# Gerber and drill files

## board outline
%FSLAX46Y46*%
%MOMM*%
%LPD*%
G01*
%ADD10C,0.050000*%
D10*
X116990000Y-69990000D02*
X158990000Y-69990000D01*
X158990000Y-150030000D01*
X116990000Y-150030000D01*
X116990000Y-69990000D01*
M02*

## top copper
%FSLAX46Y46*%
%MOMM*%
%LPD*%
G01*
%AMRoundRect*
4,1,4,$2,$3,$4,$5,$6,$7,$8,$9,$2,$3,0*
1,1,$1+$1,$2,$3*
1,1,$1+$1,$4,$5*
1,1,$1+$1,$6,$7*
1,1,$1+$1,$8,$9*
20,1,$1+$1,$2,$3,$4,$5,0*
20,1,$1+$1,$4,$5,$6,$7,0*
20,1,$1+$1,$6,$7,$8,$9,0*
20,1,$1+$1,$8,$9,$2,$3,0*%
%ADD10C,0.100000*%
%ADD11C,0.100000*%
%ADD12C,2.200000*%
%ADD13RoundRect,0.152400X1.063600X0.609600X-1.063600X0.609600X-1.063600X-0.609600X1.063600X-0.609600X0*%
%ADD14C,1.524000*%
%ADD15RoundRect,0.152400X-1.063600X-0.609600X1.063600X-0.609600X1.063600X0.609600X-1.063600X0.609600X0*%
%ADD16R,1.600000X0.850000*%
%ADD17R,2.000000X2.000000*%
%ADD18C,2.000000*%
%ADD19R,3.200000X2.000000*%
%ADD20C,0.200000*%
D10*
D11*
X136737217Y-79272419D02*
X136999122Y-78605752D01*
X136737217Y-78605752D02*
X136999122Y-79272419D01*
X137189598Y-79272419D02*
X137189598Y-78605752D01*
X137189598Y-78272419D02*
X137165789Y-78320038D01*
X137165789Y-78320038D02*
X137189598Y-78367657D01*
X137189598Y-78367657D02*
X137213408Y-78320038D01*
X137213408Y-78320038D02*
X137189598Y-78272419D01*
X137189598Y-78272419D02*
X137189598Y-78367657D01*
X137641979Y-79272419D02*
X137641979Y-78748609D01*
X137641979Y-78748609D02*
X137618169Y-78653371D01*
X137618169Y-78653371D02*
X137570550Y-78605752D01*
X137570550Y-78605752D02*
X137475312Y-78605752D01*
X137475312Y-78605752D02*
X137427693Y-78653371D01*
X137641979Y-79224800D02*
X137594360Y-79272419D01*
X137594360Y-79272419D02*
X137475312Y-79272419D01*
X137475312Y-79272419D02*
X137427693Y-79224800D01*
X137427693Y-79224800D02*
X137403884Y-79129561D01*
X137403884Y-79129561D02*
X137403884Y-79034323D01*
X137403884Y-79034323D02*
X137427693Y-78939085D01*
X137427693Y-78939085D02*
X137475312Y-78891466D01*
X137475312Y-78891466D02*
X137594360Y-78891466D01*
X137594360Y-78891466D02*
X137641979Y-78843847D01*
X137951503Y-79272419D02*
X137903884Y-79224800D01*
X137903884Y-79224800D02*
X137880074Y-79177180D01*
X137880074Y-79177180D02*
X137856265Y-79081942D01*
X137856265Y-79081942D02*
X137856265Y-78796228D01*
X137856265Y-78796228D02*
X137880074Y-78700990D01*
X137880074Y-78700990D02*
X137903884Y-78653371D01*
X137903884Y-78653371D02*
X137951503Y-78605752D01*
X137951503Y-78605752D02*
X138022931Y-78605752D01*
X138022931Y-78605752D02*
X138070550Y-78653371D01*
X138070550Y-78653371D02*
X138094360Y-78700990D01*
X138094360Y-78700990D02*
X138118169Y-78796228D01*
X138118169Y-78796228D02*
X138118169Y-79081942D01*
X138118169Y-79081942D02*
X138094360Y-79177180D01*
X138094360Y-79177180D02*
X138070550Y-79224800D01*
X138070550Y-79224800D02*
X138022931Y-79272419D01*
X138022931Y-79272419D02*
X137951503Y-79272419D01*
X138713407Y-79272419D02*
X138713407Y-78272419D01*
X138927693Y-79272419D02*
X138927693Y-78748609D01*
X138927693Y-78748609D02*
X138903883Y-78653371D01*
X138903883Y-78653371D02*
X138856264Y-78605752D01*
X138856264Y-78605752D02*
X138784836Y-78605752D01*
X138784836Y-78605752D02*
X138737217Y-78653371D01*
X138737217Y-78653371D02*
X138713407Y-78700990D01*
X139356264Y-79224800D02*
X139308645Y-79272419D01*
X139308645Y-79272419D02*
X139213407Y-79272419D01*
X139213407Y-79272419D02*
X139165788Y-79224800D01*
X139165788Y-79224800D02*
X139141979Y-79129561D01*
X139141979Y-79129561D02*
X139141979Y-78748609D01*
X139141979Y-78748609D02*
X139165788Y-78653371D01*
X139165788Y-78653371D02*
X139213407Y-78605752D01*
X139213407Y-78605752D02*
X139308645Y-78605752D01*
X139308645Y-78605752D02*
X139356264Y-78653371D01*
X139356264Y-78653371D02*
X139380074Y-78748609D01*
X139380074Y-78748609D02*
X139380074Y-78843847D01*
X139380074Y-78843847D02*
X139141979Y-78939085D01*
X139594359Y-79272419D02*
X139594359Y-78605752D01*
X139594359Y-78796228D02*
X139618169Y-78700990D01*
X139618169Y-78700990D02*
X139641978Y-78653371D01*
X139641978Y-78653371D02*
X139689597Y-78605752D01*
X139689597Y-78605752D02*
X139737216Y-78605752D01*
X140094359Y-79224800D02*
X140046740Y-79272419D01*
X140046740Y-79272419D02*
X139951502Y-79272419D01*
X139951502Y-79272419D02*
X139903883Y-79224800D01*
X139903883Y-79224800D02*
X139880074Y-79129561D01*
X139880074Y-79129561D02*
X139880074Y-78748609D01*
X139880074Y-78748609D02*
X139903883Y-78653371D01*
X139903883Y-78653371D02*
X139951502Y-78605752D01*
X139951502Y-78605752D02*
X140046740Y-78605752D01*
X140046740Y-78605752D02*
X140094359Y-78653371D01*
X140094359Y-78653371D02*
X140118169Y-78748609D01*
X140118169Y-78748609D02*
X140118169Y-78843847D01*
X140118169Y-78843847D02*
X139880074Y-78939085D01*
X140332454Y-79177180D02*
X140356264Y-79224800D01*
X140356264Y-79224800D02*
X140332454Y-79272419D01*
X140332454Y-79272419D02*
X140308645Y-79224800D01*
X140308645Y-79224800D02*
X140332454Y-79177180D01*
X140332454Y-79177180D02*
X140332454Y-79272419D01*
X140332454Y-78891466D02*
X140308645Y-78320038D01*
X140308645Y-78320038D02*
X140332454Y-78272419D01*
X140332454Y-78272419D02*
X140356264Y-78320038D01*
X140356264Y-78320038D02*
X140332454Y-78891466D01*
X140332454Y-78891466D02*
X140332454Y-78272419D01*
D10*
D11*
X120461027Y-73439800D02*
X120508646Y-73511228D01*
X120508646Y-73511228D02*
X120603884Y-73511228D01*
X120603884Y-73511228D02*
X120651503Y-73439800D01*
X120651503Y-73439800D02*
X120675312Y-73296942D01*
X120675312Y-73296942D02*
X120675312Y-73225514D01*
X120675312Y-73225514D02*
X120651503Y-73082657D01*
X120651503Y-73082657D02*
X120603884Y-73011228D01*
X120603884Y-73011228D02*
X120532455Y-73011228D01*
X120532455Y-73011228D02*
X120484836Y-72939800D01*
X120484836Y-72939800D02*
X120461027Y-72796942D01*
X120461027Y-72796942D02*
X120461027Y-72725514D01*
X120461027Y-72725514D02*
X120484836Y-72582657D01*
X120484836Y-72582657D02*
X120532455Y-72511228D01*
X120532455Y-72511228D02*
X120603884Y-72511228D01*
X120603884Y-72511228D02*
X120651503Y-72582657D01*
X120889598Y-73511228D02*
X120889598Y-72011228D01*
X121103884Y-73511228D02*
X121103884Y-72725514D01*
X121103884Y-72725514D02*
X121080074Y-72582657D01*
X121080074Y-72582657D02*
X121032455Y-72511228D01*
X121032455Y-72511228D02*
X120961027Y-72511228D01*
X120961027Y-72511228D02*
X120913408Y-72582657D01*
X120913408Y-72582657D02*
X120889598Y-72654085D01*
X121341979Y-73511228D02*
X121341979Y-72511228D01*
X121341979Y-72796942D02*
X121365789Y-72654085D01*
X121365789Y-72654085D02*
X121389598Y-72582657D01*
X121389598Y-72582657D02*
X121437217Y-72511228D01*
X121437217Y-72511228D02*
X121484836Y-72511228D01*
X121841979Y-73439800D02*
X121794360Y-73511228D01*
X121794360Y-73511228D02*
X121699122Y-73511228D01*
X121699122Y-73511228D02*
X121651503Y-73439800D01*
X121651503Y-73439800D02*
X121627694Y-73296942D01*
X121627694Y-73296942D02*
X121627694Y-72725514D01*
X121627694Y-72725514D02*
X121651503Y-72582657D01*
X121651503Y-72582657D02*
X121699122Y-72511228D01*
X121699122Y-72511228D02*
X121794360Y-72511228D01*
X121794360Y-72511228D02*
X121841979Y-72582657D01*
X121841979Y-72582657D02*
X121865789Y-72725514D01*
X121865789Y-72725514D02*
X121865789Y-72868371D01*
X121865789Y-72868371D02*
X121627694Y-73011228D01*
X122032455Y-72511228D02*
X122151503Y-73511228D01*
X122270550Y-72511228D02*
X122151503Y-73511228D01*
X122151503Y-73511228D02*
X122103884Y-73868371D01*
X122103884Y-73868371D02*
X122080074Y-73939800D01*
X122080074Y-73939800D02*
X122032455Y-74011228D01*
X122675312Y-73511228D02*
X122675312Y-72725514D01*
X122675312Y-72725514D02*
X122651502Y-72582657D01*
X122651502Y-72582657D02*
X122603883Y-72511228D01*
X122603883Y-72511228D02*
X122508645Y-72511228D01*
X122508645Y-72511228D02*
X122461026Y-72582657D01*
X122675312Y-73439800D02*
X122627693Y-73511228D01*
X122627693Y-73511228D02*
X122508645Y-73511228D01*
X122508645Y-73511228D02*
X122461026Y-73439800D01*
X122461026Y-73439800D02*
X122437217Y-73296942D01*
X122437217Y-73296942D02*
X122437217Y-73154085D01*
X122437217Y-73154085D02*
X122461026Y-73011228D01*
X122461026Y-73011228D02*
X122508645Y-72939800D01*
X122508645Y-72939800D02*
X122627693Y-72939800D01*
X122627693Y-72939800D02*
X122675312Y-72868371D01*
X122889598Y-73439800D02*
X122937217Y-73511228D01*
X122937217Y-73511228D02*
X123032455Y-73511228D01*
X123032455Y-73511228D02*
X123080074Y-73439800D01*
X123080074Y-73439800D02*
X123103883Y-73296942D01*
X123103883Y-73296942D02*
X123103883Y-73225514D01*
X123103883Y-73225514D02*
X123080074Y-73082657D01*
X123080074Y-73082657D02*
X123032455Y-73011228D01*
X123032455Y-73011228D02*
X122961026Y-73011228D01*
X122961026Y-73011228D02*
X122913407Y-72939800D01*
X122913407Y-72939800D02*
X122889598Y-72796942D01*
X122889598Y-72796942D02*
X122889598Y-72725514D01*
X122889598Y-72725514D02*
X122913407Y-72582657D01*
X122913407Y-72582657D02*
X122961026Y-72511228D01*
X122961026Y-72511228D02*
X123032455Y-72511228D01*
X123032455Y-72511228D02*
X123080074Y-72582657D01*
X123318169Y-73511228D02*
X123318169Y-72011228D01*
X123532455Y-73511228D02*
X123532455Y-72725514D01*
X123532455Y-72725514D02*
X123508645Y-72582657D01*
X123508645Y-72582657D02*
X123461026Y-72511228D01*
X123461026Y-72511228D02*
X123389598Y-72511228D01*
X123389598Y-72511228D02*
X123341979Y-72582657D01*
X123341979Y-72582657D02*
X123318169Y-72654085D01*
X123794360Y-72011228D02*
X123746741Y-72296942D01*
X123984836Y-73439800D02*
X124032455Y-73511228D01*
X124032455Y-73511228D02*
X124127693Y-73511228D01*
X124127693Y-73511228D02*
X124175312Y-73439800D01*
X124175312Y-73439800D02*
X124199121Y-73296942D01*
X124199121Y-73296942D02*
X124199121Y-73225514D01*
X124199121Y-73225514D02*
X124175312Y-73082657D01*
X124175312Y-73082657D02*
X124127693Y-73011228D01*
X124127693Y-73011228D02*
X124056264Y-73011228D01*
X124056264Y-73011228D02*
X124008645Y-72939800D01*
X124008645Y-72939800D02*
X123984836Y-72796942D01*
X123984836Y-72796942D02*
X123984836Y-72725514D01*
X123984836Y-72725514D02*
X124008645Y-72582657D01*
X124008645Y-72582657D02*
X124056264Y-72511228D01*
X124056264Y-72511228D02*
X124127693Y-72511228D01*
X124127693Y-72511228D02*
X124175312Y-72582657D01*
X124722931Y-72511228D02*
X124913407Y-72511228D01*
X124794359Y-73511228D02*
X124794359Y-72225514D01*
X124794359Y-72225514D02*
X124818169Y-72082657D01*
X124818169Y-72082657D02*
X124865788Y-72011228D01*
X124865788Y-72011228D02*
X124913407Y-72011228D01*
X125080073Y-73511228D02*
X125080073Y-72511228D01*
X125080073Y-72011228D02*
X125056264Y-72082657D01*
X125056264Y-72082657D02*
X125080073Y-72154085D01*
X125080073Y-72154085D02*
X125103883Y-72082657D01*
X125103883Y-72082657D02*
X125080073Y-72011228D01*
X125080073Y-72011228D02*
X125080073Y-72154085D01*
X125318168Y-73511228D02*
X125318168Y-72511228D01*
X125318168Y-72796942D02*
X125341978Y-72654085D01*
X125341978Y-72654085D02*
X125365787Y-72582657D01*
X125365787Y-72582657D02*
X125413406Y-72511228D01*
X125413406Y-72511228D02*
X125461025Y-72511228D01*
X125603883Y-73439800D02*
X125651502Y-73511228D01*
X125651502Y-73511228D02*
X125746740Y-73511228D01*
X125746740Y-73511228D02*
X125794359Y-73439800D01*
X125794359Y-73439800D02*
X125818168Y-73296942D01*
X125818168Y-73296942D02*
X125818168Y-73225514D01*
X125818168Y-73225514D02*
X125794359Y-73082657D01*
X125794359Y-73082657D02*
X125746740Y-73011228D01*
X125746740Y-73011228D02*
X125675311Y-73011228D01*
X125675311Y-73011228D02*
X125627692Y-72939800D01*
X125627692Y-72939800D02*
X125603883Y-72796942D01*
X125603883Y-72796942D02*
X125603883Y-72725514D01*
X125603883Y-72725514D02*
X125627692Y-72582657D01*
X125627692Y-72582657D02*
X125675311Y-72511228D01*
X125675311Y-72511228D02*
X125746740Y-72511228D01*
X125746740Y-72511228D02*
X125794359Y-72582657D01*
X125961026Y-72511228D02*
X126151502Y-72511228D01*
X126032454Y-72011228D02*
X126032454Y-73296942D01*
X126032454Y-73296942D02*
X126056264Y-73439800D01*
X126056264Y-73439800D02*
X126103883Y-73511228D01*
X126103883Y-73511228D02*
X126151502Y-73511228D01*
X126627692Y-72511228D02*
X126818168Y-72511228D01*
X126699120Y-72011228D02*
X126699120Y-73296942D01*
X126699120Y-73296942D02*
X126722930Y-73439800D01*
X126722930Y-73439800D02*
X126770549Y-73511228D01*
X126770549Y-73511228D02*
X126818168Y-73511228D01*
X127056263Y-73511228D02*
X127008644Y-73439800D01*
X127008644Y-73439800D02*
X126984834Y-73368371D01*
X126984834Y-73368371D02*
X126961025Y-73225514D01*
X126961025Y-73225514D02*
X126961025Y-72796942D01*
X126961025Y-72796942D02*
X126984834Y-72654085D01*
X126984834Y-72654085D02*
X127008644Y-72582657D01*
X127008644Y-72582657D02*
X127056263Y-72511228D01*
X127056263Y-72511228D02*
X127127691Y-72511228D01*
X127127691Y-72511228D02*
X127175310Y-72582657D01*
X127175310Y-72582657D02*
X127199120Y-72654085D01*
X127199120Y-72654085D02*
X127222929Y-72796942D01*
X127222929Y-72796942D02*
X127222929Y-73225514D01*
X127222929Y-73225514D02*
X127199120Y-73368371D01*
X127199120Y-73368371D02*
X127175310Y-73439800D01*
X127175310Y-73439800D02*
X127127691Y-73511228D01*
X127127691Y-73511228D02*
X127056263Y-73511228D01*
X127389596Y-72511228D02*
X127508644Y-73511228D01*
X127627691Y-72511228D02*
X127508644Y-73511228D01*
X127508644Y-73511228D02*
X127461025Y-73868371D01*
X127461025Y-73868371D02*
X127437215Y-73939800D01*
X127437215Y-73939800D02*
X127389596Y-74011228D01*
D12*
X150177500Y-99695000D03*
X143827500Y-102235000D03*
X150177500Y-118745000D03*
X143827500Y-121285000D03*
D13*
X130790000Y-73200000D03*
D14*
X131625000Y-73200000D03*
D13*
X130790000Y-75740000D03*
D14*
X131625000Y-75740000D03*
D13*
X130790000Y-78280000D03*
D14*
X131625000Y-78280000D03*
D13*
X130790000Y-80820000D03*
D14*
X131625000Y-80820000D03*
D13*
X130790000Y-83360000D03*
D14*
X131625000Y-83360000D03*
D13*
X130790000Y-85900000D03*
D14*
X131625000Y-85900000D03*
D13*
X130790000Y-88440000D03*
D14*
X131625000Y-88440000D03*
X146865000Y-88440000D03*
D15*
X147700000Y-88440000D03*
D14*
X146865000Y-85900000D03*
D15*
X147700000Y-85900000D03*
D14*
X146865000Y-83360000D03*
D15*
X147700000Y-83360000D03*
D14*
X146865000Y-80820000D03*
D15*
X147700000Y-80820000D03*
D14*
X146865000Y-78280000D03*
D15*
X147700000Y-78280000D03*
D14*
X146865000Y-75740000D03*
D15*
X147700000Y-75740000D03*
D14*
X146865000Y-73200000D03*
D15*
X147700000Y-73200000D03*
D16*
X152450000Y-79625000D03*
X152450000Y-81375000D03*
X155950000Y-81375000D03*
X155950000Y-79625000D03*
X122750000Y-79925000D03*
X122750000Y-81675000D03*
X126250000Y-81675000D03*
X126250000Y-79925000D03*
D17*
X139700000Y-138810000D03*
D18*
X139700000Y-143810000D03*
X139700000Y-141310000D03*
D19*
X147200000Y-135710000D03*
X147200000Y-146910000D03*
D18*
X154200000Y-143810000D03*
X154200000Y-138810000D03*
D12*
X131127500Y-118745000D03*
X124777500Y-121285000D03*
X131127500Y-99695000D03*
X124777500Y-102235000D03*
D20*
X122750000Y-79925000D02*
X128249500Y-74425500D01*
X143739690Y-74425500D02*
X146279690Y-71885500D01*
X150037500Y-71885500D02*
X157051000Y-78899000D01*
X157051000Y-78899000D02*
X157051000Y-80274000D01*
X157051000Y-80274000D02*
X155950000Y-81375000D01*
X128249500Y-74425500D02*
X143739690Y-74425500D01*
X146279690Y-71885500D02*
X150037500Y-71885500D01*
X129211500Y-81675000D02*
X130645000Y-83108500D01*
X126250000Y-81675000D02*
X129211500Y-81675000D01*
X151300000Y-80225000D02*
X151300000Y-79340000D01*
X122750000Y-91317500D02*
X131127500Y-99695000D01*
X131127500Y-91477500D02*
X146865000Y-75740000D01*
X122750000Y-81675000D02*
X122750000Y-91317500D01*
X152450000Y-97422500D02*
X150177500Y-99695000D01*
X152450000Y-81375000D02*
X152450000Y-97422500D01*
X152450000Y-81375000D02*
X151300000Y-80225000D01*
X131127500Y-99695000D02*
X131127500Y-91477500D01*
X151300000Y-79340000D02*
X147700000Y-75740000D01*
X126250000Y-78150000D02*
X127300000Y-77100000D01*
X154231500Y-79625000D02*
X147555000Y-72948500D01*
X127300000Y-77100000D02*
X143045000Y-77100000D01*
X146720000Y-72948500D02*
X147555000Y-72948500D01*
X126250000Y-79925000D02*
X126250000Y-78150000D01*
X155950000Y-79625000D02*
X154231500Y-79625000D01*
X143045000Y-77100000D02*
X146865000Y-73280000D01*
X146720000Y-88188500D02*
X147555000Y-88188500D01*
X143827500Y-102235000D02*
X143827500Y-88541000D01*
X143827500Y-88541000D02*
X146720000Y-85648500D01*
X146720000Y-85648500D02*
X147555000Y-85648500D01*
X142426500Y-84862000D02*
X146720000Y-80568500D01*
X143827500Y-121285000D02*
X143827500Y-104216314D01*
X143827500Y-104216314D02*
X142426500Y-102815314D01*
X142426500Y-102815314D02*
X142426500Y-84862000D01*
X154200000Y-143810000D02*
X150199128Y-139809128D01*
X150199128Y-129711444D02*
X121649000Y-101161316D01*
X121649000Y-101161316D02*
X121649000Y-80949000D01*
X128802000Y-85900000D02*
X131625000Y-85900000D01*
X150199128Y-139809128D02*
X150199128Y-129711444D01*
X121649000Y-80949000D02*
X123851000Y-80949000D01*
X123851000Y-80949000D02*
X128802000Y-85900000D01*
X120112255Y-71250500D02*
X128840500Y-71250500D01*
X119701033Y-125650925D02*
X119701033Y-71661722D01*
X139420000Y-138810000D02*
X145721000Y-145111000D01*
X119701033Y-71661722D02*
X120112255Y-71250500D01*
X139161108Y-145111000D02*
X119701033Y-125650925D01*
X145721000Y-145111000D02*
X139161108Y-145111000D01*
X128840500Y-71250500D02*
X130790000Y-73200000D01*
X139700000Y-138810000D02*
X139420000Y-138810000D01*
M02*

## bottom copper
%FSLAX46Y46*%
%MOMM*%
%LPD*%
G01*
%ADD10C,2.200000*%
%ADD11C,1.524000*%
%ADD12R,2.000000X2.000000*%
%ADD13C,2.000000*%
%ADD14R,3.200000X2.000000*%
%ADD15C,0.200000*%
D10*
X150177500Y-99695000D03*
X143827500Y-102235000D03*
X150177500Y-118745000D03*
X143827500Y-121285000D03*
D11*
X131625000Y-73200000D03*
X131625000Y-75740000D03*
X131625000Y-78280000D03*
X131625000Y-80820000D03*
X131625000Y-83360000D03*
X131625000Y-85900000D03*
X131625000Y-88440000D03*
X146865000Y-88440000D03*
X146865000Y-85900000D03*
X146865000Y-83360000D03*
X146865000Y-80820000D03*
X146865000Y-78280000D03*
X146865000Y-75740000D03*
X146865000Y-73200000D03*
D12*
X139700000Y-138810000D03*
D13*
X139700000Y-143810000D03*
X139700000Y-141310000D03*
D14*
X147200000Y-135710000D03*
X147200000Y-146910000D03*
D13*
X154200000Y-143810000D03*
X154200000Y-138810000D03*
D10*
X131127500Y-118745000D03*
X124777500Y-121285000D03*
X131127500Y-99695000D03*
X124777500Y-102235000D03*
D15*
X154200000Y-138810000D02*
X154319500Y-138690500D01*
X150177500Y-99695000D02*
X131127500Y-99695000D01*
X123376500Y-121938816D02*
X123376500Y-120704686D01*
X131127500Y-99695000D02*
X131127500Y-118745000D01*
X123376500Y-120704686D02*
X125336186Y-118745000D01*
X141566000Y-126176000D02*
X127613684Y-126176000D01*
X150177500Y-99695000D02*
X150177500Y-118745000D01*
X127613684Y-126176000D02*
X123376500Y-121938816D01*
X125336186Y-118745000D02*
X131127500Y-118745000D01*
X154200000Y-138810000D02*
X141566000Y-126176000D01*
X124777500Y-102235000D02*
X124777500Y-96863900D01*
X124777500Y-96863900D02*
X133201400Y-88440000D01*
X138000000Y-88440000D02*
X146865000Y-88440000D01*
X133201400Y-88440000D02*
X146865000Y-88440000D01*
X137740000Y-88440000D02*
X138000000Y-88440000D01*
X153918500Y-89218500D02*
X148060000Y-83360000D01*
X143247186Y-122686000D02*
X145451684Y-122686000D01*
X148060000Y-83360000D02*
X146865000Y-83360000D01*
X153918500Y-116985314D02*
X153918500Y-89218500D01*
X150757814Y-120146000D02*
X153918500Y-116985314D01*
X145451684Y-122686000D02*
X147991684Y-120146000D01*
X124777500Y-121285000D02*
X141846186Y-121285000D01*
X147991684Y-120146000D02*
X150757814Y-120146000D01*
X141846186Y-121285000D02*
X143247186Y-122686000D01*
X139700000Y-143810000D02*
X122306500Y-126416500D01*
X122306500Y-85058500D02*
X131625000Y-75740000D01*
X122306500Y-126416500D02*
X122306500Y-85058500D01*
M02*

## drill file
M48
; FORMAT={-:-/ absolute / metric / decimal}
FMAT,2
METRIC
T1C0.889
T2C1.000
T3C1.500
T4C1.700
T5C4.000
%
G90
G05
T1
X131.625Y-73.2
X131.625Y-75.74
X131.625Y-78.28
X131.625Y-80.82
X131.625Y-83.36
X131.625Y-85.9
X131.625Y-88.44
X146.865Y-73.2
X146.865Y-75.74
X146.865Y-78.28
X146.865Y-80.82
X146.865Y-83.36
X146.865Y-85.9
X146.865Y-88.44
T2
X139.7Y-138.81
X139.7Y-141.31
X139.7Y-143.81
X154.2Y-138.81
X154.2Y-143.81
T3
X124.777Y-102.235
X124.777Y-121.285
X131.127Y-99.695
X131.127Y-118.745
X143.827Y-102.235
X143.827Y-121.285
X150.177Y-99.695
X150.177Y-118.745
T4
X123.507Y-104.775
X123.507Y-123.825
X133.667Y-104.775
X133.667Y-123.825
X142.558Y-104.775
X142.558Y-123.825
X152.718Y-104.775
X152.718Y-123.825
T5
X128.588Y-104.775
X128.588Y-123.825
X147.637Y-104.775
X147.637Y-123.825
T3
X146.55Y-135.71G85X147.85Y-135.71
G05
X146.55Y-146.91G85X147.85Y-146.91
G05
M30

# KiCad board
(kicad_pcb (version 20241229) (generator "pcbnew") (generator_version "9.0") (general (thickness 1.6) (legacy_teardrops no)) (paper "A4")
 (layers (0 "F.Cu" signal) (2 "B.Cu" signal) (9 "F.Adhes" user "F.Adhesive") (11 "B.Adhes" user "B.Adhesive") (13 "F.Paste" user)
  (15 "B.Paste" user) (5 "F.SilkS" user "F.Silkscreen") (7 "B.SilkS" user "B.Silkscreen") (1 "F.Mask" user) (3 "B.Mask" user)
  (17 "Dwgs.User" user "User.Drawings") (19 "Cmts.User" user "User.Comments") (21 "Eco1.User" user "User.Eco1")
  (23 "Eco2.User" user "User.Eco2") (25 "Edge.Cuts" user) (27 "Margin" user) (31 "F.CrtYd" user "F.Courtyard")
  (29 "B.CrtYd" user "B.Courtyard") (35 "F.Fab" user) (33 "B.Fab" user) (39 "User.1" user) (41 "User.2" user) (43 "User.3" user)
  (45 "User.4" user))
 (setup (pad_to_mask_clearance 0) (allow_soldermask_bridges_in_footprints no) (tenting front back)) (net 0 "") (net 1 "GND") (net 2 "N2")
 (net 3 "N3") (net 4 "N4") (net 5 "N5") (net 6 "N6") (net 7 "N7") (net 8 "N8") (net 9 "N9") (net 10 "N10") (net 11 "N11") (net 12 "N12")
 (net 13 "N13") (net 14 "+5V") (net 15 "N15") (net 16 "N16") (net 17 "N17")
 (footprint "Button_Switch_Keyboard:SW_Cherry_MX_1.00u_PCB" (layer "F.Cu") (at 150.1775 99.695)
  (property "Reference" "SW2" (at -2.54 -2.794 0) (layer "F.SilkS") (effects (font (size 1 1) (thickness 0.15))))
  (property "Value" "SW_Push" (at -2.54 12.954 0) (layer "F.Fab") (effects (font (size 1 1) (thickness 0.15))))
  (pad "" np_thru_hole circle (at -7.62 5.08) (size 1.7 1.7) (drill 1.7) (layers "*.Cu" "*.Mask"))
  (pad "" np_thru_hole circle (at -2.54 5.08) (size 4 4) (drill 4) (layers "*.Cu" "*.Mask"))
  (pad "" np_thru_hole circle (at 2.54 5.08) (size 1.7 1.7) (drill 1.7) (layers "*.Cu" "*.Mask"))
  (pad "1" thru_hole circle (at 0 0) (size 2.2 2.2) (drill 1.5) (layers "*.Cu" "*.Mask") (remove_unused_layers no) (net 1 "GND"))
  (pad "2" thru_hole circle (at -6.35 2.54) (size 2.2 2.2) (drill 1.5) (layers "*.Cu" "*.Mask") (remove_unused_layers no) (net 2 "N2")))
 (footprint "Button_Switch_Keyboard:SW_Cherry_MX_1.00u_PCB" (layer "F.Cu") (at 150.1775 118.745)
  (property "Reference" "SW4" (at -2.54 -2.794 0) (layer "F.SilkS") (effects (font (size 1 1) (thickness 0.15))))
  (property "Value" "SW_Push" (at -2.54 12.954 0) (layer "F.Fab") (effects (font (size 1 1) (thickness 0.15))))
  (pad "" np_thru_hole circle (at -7.62 5.08) (size 1.7 1.7) (drill 1.7) (layers "*.Cu" "*.Mask"))
  (pad "" np_thru_hole circle (at -2.54 5.08) (size 4 4) (drill 4) (layers "*.Cu" "*.Mask"))
  (pad "" np_thru_hole circle (at 2.54 5.08) (size 1.7 1.7) (drill 1.7) (layers "*.Cu" "*.Mask"))
  (pad "1" thru_hole circle (at 0 0) (size 2.2 2.2) (drill 1.5) (layers "*.Cu" "*.Mask") (remove_unused_layers no) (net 1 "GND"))
  (pad "2" thru_hole circle (at -6.35 2.54) (size 2.2 2.2) (drill 1.5) (layers "*.Cu" "*.Mask") (remove_unused_layers no) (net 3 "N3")))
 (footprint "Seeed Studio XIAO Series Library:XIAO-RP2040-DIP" (layer "F.Cu") (at 139.245 80.82)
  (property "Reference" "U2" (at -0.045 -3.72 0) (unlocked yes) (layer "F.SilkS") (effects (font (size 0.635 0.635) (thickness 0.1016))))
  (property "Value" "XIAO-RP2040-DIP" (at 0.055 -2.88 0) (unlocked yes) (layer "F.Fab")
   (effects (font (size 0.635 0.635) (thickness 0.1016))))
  (pad "1" smd roundrect (at -8.455 -7.62 180) (size 2.432 1.524) (layers "F.Cu" "F.Mask") (roundrect_rratio 0.1) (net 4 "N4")
   (thermal_bridge_angle 45))
  (pad "1" thru_hole circle (at -7.62 -7.62 180) (size 1.524 1.524) (drill 0.889) (layers "*.Cu" "*.Mask") (remove_unused_layers no)
   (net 4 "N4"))
  (pad "2" smd roundrect (at -8.455 -5.08 180) (size 2.432 1.524) (layers "F.Cu" "F.Mask") (roundrect_rratio 0.1) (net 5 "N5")
   (thermal_bridge_angle 45))
  (pad "2" thru_hole circle (at -7.62 -5.08 180) (size 1.524 1.524) (drill 0.889) (layers "*.Cu" "*.Mask") (remove_unused_layers no)
   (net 5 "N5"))
  (pad "3" smd roundrect (at -8.455 -2.54 180) (size 2.432 1.524) (layers "F.Cu" "F.Mask") (roundrect_rratio 0.1) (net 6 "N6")
   (thermal_bridge_angle 45))
  (pad "3" thru_hole circle (at -7.62 -2.54 180) (size 1.524 1.524) (drill 0.889) (layers "*.Cu" "*.Mask") (remove_unused_layers no)
   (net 6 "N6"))
  (pad "4" smd roundrect (at -8.455 0 180) (size 2.432 1.524) (layers "F.Cu" "F.Mask") (roundrect_rratio 0.1) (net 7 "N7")
   (thermal_bridge_angle 45))
  (pad "4" thru_hole circle (at -7.62 0 180) (size 1.524 1.524) (drill 0.889) (layers "*.Cu" "*.Mask") (remove_unused_layers no)
   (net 7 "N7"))
  (pad "5" smd roundrect (at -8.455 2.54 180) (size 2.432 1.524) (layers "F.Cu" "F.Mask") (roundrect_rratio 0.1) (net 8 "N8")
   (thermal_bridge_angle 45))
  (pad "5" thru_hole circle (at -7.62 2.54 180) (size 1.524 1.524) (drill 0.889) (layers "*.Cu" "*.Mask") (remove_unused_layers no)
   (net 8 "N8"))
  (pad "6" smd roundrect (at -8.455 5.08 180) (size 2.432 1.524) (layers "F.Cu" "F.Mask") (roundrect_rratio 0.1) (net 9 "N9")
   (thermal_bridge_angle 45))
  (pad "6" thru_hole circle (at -7.62 5.08 180) (size 1.524 1.524) (drill 0.889) (layers "*.Cu" "*.Mask") (remove_unused_layers no)
   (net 9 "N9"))
  (pad "7" smd roundrect (at -8.455 7.62 180) (size 2.432 1.524) (layers "F.Cu" "F.Mask") (roundrect_rratio 0.1) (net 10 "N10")
   (thermal_bridge_angle 45))
  (pad "7" thru_hole circle (at -7.62 7.62 180) (size 1.524 1.524) (drill 0.889) (layers "*.Cu" "*.Mask") (remove_unused_layers no)
   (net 10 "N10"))
  (pad "8" thru_hole circle (at 7.62 7.62) (size 1.524 1.524) (drill 0.889) (layers "*.Cu" "*.Mask") (remove_unused_layers no)
   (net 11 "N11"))
  (pad "8" smd roundrect (at 8.455 7.62) (size 2.432 1.524) (layers "F.Cu" "F.Mask") (roundrect_rratio 0.1) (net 11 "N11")
   (thermal_bridge_angle 45))
  (pad "9" thru_hole circle (at 7.62 5.08) (size 1.524 1.524) (drill 0.889) (layers "*.Cu" "*.Mask") (remove_unused_layers no) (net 2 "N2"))
  (pad "9" smd roundrect (at 8.455 5.08) (size 2.432 1.524) (layers "F.Cu" "F.Mask") (roundrect_rratio 0.1) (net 2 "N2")
   (thermal_bridge_angle 45))
  (pad "10" thru_hole circle (at 7.62 2.54) (size 1.524 1.524) (drill 0.889) (layers "*.Cu" "*.Mask") (remove_unused_layers no)
   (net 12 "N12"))
  (pad "10" smd roundrect (at 8.455 2.54) (size 2.432 1.524) (layers "F.Cu" "F.Mask") (roundrect_rratio 0.1) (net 12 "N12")
   (thermal_bridge_angle 45))
  (pad "11" thru_hole circle (at 7.62 0) (size 1.524 1.524) (drill 0.889) (layers "*.Cu" "*.Mask") (remove_unused_layers no) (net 3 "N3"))
  (pad "11" smd roundrect (at 8.455 0) (size 2.432 1.524) (layers "F.Cu" "F.Mask") (roundrect_rratio 0.1) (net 3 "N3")
   (thermal_bridge_angle 45))
  (pad "12" thru_hole circle (at 7.62 -2.54) (size 1.524 1.524) (drill 0.889) (layers "*.Cu" "*.Mask") (remove_unused_layers no)
   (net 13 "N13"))
  (pad "12" smd roundrect (at 8.455 -2.54) (size 2.432 1.524) (layers "F.Cu" "F.Mask") (roundrect_rratio 0.1) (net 13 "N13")
   (thermal_bridge_angle 45))
  (pad "13" thru_hole circle (at 7.62 -5.08) (size 1.524 1.524) (drill 0.889) (layers "*.Cu" "*.Mask") (remove_unused_layers no)
   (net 1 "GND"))
  (pad "13" smd roundrect (at 8.455 -5.08) (size 2.432 1.524) (layers "F.Cu" "F.Mask") (roundrect_rratio 0.1) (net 1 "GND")
   (thermal_bridge_angle 45))
  (pad "14" thru_hole circle (at 7.62 -7.62) (size 1.524 1.524) (drill 0.889) (layers "*.Cu" "*.Mask") (remove_unused_layers no)
   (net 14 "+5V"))
  (pad "14" smd roundrect (at 8.455 -7.62) (size 2.432 1.524) (layers "F.Cu" "F.Mask") (roundrect_rratio 0.1) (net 14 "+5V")
   (thermal_bridge_angle 45)))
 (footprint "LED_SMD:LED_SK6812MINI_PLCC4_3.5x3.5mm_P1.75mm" (layer "F.Cu") (at 154.2 80.5)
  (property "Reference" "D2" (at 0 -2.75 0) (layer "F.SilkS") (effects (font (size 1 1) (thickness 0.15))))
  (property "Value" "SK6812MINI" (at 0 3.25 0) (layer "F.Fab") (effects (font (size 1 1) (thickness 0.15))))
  (pad "1" smd rect (at -1.75 -0.875) (size 1.6 0.85) (layers "F.Cu" "F.Mask" "F.Paste") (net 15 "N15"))
  (pad "2" smd rect (at -1.75 0.875) (size 1.6 0.85) (layers "F.Cu" "F.Mask" "F.Paste") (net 1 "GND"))
  (pad "3" smd rect (at 1.75 0.875) (size 1.6 0.85) (layers "F.Cu" "F.Mask" "F.Paste") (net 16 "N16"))
  (pad "4" smd rect (at 1.75 -0.875) (size 1.6 0.85) (layers "F.Cu" "F.Mask" "F.Paste") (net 14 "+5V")))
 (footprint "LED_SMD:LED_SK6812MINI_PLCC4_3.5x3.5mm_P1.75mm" (layer "F.Cu") (at 124.5 80.8)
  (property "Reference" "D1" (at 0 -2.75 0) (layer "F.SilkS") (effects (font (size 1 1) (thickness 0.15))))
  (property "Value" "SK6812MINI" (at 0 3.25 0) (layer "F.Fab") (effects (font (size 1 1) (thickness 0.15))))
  (pad "1" smd rect (at -1.75 -0.875) (size 1.6 0.85) (layers "F.Cu" "F.Mask" "F.Paste") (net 16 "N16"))
  (pad "2" smd rect (at -1.75 0.875) (size 1.6 0.85) (layers "F.Cu" "F.Mask" "F.Paste") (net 1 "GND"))
  (pad "3" smd rect (at 1.75 0.875) (size 1.6 0.85) (layers "F.Cu" "F.Mask" "F.Paste") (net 8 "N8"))
  (pad "4" smd rect (at 1.75 -0.875) (size 1.6 0.85) (layers "F.Cu" "F.Mask" "F.Paste") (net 14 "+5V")))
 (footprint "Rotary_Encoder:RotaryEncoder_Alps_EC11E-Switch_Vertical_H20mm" (layer "F.Cu") (at 139.7 138.81)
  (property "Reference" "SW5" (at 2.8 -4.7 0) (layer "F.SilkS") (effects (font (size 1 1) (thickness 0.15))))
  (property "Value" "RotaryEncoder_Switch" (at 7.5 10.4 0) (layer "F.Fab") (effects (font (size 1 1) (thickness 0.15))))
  (pad "A" thru_hole rect (at 0 0) (size 2 2) (drill 1) (layers "*.Cu" "*.Mask") (remove_unused_layers no) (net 4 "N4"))
  (pad "B" thru_hole circle (at 0 5) (size 2 2) (drill 1) (layers "*.Cu" "*.Mask") (remove_unused_layers no) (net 5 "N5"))
  (pad "C" thru_hole circle (at 0 2.5) (size 2 2) (drill 1) (layers "*.Cu" "*.Mask") (remove_unused_layers no) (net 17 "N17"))
  (pad "MP" thru_hole rect (at 7.5 -3.1) (size 3.2 2) (drill oval 2.8 1.5) (layers "*.Cu" "*.Mask") (remove_unused_layers no))
  (pad "MP" thru_hole rect (at 7.5 8.1) (size 3.2 2) (drill oval 2.8 1.5) (layers "*.Cu" "*.Mask") (remove_unused_layers no))
  (pad "S1" thru_hole circle (at 14.5 5) (size 2 2) (drill 1) (layers "*.Cu" "*.Mask") (remove_unused_layers no) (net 9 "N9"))
  (pad "S2" thru_hole circle (at 14.5 0) (size 2 2) (drill 1) (layers "*.Cu" "*.Mask") (remove_unused_layers no) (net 1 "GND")))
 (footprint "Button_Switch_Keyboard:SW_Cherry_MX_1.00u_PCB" (layer "F.Cu") (at 131.1275 118.745)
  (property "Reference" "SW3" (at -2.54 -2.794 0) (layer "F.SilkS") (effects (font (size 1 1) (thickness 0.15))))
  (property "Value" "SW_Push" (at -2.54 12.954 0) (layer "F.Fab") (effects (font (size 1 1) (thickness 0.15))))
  (pad "" np_thru_hole circle (at -7.62 5.08) (size 1.7 1.7) (drill 1.7) (layers "*.Cu" "*.Mask"))
  (pad "" np_thru_hole circle (at -2.54 5.08) (size 4 4) (drill 4) (layers "*.Cu" "*.Mask"))
  (pad "" np_thru_hole circle (at 2.54 5.08) (size 1.7 1.7) (drill 1.7) (layers "*.Cu" "*.Mask"))
  (pad "1" thru_hole circle (at 0 0) (size 2.2 2.2) (drill 1.5) (layers "*.Cu" "*.Mask") (remove_unused_layers no) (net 1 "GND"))
  (pad "2" thru_hole circle (at -6.35 2.54) (size 2.2 2.2) (drill 1.5) (layers "*.Cu" "*.Mask") (remove_unused_layers no) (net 12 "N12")))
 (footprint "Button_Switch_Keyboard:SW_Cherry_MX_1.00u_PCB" (layer "F.Cu") (at 131.1275 99.695)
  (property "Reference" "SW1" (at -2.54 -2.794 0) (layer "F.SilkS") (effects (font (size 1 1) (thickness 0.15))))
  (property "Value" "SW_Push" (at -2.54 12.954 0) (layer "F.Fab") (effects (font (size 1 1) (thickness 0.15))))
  (pad "" np_thru_hole circle (at -7.62 5.08) (size 1.7 1.7) (drill 1.7) (layers "*.Cu" "*.Mask"))
  (pad "" np_thru_hole circle (at -2.54 5.08) (size 4 4) (drill 4) (layers "*.Cu" "*.Mask"))
  (pad "" np_thru_hole circle (at 2.54 5.08) (size 1.7 1.7) (drill 1.7) (layers "*.Cu" "*.Mask"))
  (pad "1" thru_hole circle (at 0 0) (size 2.2 2.2) (drill 1.5) (layers "*.Cu" "*.Mask") (remove_unused_layers no) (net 1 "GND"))
  (pad "2" thru_hole circle (at -6.35 2.54) (size 2.2 2.2) (drill 1.5) (layers "*.Cu" "*.Mask") (remove_unused_layers no) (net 11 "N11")))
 (gr_rect (start 116.99 69.99) (end 158.99 150.03) (stroke (width 0.05) (type default)) (fill no) (layer "Edge.Cuts"))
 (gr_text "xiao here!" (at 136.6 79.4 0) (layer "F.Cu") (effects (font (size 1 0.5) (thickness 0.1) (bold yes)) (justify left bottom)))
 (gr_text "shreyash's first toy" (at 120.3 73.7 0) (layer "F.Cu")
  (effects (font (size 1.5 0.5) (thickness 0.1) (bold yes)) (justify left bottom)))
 (segment (start 122.75 79.925) (end 128.2495 74.4255) (width 0.2) (layer "F.Cu") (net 16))
 (segment (start 143.73969 74.4255) (end 146.27969 71.8855) (width 0.2) (layer "F.Cu") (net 16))
 (segment (start 150.0375 71.8855) (end 157.051 78.899) (width 0.2) (layer "F.Cu") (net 16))
 (segment (start 157.051 78.899) (end 157.051 80.274) (width 0.2) (layer "F.Cu") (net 16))
 (segment (start 157.051 80.274) (end 155.95 81.375) (width 0.2) (layer "F.Cu") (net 16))
 (segment (start 128.2495 74.4255) (end 143.73969 74.4255) (width 0.2) (layer "F.Cu") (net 16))
 (segment (start 146.27969 71.8855) (end 150.0375 71.8855) (width 0.2) (layer "F.Cu") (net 16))
 (segment (start 129.2115 81.675) (end 130.645 83.1085) (width 0.2) (layer "F.Cu") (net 8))
 (segment (start 126.25 81.675) (end 129.2115 81.675) (width 0.2) (layer "F.Cu") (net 8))
 (segment (start 151.3 80.225) (end 151.3 79.34) (width 0.2) (layer "F.Cu") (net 1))
 (segment (start 122.75 91.3175) (end 131.1275 99.695) (width 0.2) (layer "F.Cu") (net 1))
 (segment (start 131.1275 91.4775) (end 146.865 75.74) (width 0.2) (layer "F.Cu") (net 1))
 (segment (start 122.75 81.675) (end 122.75 91.3175) (width 0.2) (layer "F.Cu") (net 1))
 (segment (start 152.45 97.4225) (end 150.1775 99.695) (width 0.2) (layer "F.Cu") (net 1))
 (segment (start 152.45 81.375) (end 152.45 97.4225) (width 0.2) (layer "F.Cu") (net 1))
 (segment (start 152.45 81.375) (end 151.3 80.225) (width 0.2) (layer "F.Cu") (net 1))
 (segment (start 131.1275 99.695) (end 131.1275 91.4775) (width 0.2) (layer "F.Cu") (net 1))
 (segment (start 151.3 79.34) (end 147.7 75.74) (width 0.2) (layer "F.Cu") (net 1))
 (segment (start 154.2 138.81) (end 154.3195 138.6905) (width 0.2) (layer "B.Cu") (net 1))
 (segment (start 150.1775 99.695) (end 131.1275 99.695) (width 0.2) (layer "B.Cu") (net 1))
 (segment (start 123.3765 121.938816) (end 123.3765 120.704686) (width 0.2) (layer "B.Cu") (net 1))
 (segment (start 131.1275 99.695) (end 131.1275 118.745) (width 0.2) (layer "B.Cu") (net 1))
 (segment (start 123.3765 120.704686) (end 125.336186 118.745) (width 0.2) (layer "B.Cu") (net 1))
 (segment (start 141.566 126.176) (end 127.613684 126.176) (width 0.2) (layer "B.Cu") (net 1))
 (segment (start 150.1775 99.695) (end 150.1775 118.745) (width 0.2) (layer "B.Cu") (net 1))
 (segment (start 127.613684 126.176) (end 123.3765 121.938816) (width 0.2) (layer "B.Cu") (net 1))
 (segment (start 125.336186 118.745) (end 131.1275 118.745) (width 0.2) (layer "B.Cu") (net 1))
 (segment (start 154.2 138.81) (end 141.566 126.176) (width 0.2) (layer "B.Cu") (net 1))
 (segment (start 126.25 78.15) (end 127.3 77.1) (width 0.2) (layer "F.Cu") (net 14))
 (segment (start 154.2315 79.625) (end 147.555 72.9485) (width 0.2) (layer "F.Cu") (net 14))
 (segment (start 127.3 77.1) (end 143.045 77.1) (width 0.2) (layer "F.Cu") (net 14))
 (segment (start 146.72 72.9485) (end 147.555 72.9485) (width 0.2) (layer "F.Cu") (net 14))
 (segment (start 126.25 79.925) (end 126.25 78.15) (width 0.2) (layer "F.Cu") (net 14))
 (segment (start 155.95 79.625) (end 154.2315 79.625) (width 0.2) (layer "F.Cu") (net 14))
 (segment (start 143.045 77.1) (end 146.865 73.28) (width 0.2) (layer "F.Cu") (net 14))
 (segment (start 146.72 88.1885) (end 147.555 88.1885) (width 0.2) (layer "F.Cu") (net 11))
 (segment (start 124.7775 102.235) (end 124.7775 96.8639) (width 0.2) (layer "B.Cu") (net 11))
 (segment (start 124.7775 96.8639) (end 133.2014 88.44) (width 0.2) (layer "B.Cu") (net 11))
 (segment (start 138 88.44) (end 146.865 88.44) (width 0.2) (layer "B.Cu") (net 11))
 (segment (start 133.2014 88.44) (end 146.865 88.44) (width 0.2) (layer "B.Cu") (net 11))
 (segment (start 137.74 88.44) (end 138 88.44) (width 0.2) (layer "B.Cu") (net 11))
 (segment (start 143.8275 102.235) (end 143.8275 88.541) (width 0.2) (layer "F.Cu") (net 2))
 (segment (start 143.8275 88.541) (end 146.72 85.6485) (width 0.2) (layer "F.Cu") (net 2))
 (segment (start 146.72 85.6485) (end 147.555 85.6485) (width 0.2) (layer "F.Cu") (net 2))
 (segment (start 153.9185 89.2185) (end 148.06 83.36) (width 0.2) (layer "B.Cu") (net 12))
 (segment (start 143.247186 122.686) (end 145.451684 122.686) (width 0.2) (layer "B.Cu") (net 12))
 (segment (start 148.06 83.36) (end 146.865 83.36) (width 0.2) (layer "B.Cu") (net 12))
 (segment (start 153.9185 116.985314) (end 153.9185 89.2185) (width 0.2) (layer "B.Cu") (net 12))
 (segment (start 150.757814 120.146) (end 153.9185 116.985314) (width 0.2) (layer "B.Cu") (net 12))
 (segment (start 145.451684 122.686) (end 147.991684 120.146) (width 0.2) (layer "B.Cu") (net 12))
 (segment (start 124.7775 121.285) (end 141.846186 121.285) (width 0.2) (layer "B.Cu") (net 12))
 (segment (start 147.991684 120.146) (end 150.757814 120.146) (width 0.2) (layer "B.Cu") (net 12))
 (segment (start 141.846186 121.285) (end 143.247186 122.686) (width 0.2) (layer "B.Cu") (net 12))
 (segment (start 142.4265 84.862) (end 146.72 80.5685) (width 0.2) (layer "F.Cu") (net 3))
 (segment (start 143.8275 121.285) (end 143.8275 104.216314) (width 0.2) (layer "F.Cu") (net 3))
 (segment (start 143.8275 104.216314) (end 142.4265 102.815314) (width 0.2) (layer "F.Cu") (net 3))
 (segment (start 142.4265 102.815314) (end 142.4265 84.862) (width 0.2) (layer "F.Cu") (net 3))
 (segment (start 154.2 143.81) (end 150.199128 139.809128) (width 0.2) (layer "F.Cu") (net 9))
 (segment (start 150.199128 129.711444) (end 121.649 101.161316) (width 0.2) (layer "F.Cu") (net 9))
 (segment (start 121.649 101.161316) (end 121.649 80.949) (width 0.2) (layer "F.Cu") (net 9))
 (segment (start 128.802 85.9) (end 131.625 85.9) (width 0.2) (layer "F.Cu") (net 9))
 (segment (start 150.199128 139.809128) (end 150.199128 129.711444) (width 0.2) (layer "F.Cu") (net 9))
 (segment (start 121.649 80.949) (end 123.851 80.949) (width 0.2) (layer "F.Cu") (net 9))
 (segment (start 123.851 80.949) (end 128.802 85.9) (width 0.2) (layer "F.Cu") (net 9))
 (segment (start 139.7 143.81) (end 122.3065 126.4165) (width 0.2) (layer "B.Cu") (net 5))
 (segment (start 122.3065 85.0585) (end 131.625 75.74) (width 0.2) (layer "B.Cu") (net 5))
 (segment (start 122.3065 126.4165) (end 122.3065 85.0585) (width 0.2) (layer "B.Cu") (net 5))
 (segment (start 120.112255 71.2505) (end 128.8405 71.2505) (width 0.2) (layer "F.Cu") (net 4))
 (segment (start 119.701033 125.650925) (end 119.701033 71.661722) (width 0.2) (layer "F.Cu") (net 4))
 (segment (start 139.42 138.81) (end 145.721 145.111) (width 0.2) (layer "F.Cu") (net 4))
 (segment (start 119.701033 71.661722) (end 120.112255 71.2505) (width 0.2) (layer "F.Cu") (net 4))
 (segment (start 139.161108 145.111) (end 119.701033 125.650925) (width 0.2) (layer "F.Cu") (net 4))
 (segment (start 145.721 145.111) (end 139.161108 145.111) (width 0.2) (layer "F.Cu") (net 4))
 (segment (start 128.8405 71.2505) (end 130.79 73.2) (width 0.2) (layer "F.Cu") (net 4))
 (segment (start 139.7 138.81) (end 139.42 138.81) (width 0.2) (layer "F.Cu") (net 4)))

